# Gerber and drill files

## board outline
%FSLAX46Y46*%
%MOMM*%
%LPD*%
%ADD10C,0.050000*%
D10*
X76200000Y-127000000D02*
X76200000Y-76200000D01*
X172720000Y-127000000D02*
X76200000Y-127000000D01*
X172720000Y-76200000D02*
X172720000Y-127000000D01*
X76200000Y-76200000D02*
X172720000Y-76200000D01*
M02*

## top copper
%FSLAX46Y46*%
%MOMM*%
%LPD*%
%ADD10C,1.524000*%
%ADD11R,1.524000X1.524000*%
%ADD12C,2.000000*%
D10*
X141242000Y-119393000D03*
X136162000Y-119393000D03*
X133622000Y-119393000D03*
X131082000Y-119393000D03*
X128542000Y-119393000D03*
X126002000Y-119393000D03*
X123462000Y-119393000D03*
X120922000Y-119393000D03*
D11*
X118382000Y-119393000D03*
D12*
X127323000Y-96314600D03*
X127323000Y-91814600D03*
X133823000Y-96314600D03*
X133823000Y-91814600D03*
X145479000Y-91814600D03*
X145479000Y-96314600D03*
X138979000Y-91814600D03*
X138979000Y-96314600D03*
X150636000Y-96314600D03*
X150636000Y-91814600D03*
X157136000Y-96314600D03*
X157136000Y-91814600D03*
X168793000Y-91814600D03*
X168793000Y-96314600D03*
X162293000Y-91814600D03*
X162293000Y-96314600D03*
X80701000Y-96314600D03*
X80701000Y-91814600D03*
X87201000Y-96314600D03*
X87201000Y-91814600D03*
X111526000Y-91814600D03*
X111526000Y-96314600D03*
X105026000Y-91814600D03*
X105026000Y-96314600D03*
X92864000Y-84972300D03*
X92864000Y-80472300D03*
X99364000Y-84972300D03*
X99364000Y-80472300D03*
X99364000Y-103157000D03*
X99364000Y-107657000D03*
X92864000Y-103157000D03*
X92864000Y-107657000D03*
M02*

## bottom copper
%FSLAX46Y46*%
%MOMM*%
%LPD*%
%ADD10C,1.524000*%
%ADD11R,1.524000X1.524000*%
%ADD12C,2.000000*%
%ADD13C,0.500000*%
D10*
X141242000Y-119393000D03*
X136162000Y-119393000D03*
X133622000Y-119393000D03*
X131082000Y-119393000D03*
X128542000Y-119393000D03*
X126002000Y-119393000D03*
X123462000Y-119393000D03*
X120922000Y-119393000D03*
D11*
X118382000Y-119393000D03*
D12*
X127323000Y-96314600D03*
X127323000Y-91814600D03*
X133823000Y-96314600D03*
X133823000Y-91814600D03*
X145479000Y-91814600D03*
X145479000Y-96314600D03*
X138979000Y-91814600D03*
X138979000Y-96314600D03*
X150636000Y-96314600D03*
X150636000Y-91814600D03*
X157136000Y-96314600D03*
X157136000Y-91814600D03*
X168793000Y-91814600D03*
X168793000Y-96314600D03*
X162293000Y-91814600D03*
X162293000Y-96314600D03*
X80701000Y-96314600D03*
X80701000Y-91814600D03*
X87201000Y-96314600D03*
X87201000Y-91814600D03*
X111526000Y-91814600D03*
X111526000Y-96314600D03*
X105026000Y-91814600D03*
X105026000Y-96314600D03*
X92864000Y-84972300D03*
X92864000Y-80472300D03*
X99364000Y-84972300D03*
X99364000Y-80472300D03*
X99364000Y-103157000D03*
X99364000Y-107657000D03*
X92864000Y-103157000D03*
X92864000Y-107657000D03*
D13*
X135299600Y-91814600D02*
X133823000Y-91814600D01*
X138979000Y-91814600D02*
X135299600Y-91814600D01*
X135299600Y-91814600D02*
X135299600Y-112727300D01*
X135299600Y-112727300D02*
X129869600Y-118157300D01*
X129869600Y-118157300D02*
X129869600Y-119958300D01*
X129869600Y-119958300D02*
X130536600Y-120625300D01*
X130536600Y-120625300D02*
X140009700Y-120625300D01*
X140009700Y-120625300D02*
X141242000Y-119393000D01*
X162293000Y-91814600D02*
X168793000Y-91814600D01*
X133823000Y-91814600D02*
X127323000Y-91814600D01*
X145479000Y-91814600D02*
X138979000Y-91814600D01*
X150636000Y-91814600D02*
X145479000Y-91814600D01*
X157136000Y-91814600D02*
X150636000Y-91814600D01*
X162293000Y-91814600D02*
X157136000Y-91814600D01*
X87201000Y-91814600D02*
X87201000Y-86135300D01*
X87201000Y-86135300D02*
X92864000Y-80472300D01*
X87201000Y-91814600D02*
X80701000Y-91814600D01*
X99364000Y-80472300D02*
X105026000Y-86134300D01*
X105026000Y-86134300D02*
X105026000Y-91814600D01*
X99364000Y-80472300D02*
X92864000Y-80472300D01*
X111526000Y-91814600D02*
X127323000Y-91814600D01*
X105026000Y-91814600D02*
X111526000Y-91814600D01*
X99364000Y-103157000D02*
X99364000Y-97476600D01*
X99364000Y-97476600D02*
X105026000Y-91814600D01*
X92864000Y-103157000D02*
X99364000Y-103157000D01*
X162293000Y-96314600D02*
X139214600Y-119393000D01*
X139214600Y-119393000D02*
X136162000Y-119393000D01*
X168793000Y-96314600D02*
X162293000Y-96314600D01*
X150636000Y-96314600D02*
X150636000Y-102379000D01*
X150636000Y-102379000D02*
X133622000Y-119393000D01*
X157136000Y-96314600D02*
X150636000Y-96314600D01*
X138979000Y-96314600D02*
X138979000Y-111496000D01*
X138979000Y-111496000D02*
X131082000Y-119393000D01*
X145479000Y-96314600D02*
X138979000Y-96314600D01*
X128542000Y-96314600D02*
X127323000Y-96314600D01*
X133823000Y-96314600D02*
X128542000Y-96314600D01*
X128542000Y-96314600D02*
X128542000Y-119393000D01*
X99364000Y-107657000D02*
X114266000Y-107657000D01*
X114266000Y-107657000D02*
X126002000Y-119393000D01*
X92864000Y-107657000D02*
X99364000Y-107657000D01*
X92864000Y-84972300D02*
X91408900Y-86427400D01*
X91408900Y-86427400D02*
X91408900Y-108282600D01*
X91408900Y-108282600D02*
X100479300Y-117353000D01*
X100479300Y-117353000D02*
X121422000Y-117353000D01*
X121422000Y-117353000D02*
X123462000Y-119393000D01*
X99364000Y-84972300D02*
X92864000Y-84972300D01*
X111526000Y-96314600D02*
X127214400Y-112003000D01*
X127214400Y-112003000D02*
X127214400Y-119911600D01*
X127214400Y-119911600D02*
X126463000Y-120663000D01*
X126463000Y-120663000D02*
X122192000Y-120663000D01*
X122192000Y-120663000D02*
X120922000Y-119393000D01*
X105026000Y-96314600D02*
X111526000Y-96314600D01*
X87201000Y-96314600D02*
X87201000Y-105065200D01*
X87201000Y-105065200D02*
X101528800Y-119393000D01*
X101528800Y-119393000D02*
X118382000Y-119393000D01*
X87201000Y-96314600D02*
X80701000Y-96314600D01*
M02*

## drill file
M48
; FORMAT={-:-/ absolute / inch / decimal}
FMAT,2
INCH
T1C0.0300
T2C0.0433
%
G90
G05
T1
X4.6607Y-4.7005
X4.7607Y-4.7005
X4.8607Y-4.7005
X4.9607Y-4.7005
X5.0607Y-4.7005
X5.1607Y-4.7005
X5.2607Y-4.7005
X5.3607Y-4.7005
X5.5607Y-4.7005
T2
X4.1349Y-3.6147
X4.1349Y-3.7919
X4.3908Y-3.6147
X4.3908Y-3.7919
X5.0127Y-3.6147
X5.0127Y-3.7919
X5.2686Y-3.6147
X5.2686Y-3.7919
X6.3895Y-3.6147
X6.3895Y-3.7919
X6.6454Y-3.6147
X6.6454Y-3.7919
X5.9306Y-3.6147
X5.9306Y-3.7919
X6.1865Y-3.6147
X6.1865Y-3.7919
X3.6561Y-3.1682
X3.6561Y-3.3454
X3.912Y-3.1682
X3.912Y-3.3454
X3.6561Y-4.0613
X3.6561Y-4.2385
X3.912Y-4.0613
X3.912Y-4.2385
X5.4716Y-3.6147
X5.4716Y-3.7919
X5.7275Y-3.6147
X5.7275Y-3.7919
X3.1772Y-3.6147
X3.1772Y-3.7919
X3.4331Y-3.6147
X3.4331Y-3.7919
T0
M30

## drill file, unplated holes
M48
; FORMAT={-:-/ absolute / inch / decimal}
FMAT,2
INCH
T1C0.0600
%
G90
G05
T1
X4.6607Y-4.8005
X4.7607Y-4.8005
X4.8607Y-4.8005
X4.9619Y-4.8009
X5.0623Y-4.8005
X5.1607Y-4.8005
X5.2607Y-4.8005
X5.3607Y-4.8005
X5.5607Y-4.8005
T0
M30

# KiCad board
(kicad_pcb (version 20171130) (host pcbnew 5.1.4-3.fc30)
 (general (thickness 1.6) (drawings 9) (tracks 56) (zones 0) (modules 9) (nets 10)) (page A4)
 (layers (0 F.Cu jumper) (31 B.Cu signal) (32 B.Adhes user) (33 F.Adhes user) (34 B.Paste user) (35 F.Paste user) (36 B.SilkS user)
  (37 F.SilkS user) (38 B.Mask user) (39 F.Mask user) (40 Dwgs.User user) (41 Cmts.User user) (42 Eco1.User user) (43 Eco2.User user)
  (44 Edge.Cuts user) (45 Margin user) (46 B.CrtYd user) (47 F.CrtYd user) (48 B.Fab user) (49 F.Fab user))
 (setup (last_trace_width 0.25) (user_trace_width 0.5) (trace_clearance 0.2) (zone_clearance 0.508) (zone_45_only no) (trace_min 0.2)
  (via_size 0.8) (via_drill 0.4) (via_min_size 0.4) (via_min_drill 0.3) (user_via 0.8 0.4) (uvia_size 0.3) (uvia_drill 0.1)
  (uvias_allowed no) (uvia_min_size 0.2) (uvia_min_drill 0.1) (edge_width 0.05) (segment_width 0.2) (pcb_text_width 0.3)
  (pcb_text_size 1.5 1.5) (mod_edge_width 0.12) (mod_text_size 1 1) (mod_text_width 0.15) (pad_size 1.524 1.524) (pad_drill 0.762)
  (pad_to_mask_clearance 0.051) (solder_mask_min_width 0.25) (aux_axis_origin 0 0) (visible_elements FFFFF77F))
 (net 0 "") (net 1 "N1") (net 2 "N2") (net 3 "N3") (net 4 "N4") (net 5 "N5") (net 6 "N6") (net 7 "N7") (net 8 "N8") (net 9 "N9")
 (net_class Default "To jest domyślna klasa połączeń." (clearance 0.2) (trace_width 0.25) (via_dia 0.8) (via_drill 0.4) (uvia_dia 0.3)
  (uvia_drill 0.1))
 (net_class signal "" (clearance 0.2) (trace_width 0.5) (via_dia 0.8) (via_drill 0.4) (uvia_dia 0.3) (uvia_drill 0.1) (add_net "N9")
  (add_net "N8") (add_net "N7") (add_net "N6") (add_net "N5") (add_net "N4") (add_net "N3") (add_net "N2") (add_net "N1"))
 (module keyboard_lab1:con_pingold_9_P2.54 (layer F.Cu) (at 118.382 119.393)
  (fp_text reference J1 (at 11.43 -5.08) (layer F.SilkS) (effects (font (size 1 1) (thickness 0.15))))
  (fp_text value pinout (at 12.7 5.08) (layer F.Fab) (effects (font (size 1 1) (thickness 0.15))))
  (pad "" np_thru_hole circle (at 22.86 2.54) (size 1.524 1.524) (drill 1.524) (layers *.Cu *.Mask))
  (pad "" np_thru_hole circle (at 17.78 2.54) (size 1.524 1.524) (drill 1.524) (layers *.Cu *.Mask))
  (pad "" np_thru_hole circle (at 15.24 2.54) (size 1.524 1.524) (drill 1.524) (layers *.Cu *.Mask))
  (pad "" np_thru_hole circle (at 12.7 2.54) (size 1.524 1.524) (drill 1.524) (layers *.Cu *.Mask))
  (pad "" np_thru_hole circle (at 10.2 2.54) (size 1.524 1.524) (drill 1.524) (layers *.Cu *.Mask))
  (pad "" np_thru_hole circle (at 7.65 2.55) (size 1.524 1.524) (drill 1.524) (layers *.Cu *.Mask))
  (pad "" np_thru_hole circle (at 5.08 2.54) (size 1.524 1.524) (drill 1.524) (layers *.Cu *.Mask))
  (pad "" np_thru_hole circle (at 2.54 2.54) (size 1.524 1.524) (drill 1.524) (layers *.Cu *.Mask))
  (pad "" np_thru_hole circle (at 0 2.54) (size 1.524 1.524) (drill 1.524) (layers *.Cu *.Mask))
  (pad 9 thru_hole circle (at 22.86 0) (size 1.524 1.524) (drill 0.762) (layers *.Cu *.Mask) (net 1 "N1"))
  (pad 8 thru_hole circle (at 17.78 0) (size 1.524 1.524) (drill 0.762) (layers *.Cu *.Mask) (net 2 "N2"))
  (pad 7 thru_hole circle (at 15.24 0) (size 1.524 1.524) (drill 0.762) (layers *.Cu *.Mask) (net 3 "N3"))
  (pad 6 thru_hole circle (at 12.7 0) (size 1.524 1.524) (drill 0.762) (layers *.Cu *.Mask) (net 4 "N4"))
  (pad 5 thru_hole circle (at 10.16 0) (size 1.524 1.524) (drill 0.762) (layers *.Cu *.Mask) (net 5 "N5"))
  (pad 4 thru_hole circle (at 7.62 0) (size 1.524 1.524) (drill 0.762) (layers *.Cu *.Mask) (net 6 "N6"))
  (pad 3 thru_hole circle (at 5.08 0) (size 1.524 1.524) (drill 0.762) (layers *.Cu *.Mask) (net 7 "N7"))
  (pad 2 thru_hole circle (at 2.54 0) (size 1.524 1.524) (drill 0.762) (layers *.Cu *.Mask) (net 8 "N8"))
  (pad 1 thru_hole rect (at 0 0) (size 1.524 1.524) (drill 0.762) (layers *.Cu *.Mask) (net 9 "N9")))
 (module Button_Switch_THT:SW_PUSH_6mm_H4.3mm (layer F.Cu) (at 127.323 91.8146)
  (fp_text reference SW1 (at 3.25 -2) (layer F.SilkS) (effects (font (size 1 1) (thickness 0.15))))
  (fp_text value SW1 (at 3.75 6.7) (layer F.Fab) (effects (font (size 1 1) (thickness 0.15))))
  (pad 2 thru_hole circle (at 0 4.5 90) (size 2 2) (drill 1.1) (layers *.Cu *.Mask) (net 5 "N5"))
  (pad 1 thru_hole circle (at 0 0 90) (size 2 2) (drill 1.1) (layers *.Cu *.Mask) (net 1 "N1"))
  (pad 2 thru_hole circle (at 6.5 4.5 90) (size 2 2) (drill 1.1) (layers *.Cu *.Mask) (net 5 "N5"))
  (pad 1 thru_hole circle (at 6.5 0 90) (size 2 2) (drill 1.1) (layers *.Cu *.Mask) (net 1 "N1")))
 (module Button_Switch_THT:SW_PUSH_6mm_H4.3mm (layer F.Cu) (at 138.979 91.8146)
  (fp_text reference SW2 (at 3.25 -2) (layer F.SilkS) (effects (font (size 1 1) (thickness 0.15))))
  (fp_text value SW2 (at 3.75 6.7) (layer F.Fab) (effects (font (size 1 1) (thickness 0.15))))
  (pad 1 thru_hole circle (at 6.5 0 90) (size 2 2) (drill 1.1) (layers *.Cu *.Mask) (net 1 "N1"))
  (pad 2 thru_hole circle (at 6.5 4.5 90) (size 2 2) (drill 1.1) (layers *.Cu *.Mask) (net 4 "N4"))
  (pad 1 thru_hole circle (at 0 0 90) (size 2 2) (drill 1.1) (layers *.Cu *.Mask) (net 1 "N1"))
  (pad 2 thru_hole circle (at 0 4.5 90) (size 2 2) (drill 1.1) (layers *.Cu *.Mask) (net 4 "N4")))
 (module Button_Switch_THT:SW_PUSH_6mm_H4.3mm (layer F.Cu) (at 150.636 91.8146)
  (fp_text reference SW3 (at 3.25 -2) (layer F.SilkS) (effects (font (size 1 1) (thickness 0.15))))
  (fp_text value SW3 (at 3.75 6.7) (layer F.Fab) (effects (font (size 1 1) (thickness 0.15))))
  (pad 2 thru_hole circle (at 0 4.5 90) (size 2 2) (drill 1.1) (layers *.Cu *.Mask) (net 3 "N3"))
  (pad 1 thru_hole circle (at 0 0 90) (size 2 2) (drill 1.1) (layers *.Cu *.Mask) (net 1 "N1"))
  (pad 2 thru_hole circle (at 6.5 4.5 90) (size 2 2) (drill 1.1) (layers *.Cu *.Mask) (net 3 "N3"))
  (pad 1 thru_hole circle (at 6.5 0 90) (size 2 2) (drill 1.1) (layers *.Cu *.Mask) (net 1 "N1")))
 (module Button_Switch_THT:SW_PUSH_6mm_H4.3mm (layer F.Cu) (at 162.293 91.8146)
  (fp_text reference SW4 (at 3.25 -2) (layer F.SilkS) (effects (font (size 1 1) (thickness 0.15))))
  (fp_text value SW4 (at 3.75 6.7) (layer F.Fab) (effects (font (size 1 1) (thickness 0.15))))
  (pad 1 thru_hole circle (at 6.5 0 90) (size 2 2) (drill 1.1) (layers *.Cu *.Mask) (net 1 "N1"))
  (pad 2 thru_hole circle (at 6.5 4.5 90) (size 2 2) (drill 1.1) (layers *.Cu *.Mask) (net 2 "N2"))
  (pad 1 thru_hole circle (at 0 0 90) (size 2 2) (drill 1.1) (layers *.Cu *.Mask) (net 1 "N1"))
  (pad 2 thru_hole circle (at 0 4.5 90) (size 2 2) (drill 1.1) (layers *.Cu *.Mask) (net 2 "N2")))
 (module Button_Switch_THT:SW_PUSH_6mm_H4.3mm (layer F.Cu) (at 80.701 91.8146)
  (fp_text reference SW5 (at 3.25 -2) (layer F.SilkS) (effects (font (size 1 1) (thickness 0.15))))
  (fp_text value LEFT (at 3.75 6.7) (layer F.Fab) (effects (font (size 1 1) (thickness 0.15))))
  (pad 2 thru_hole circle (at 0 4.5 90) (size 2 2) (drill 1.1) (layers *.Cu *.Mask) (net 9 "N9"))
  (pad 1 thru_hole circle (at 0 0 90) (size 2 2) (drill 1.1) (layers *.Cu *.Mask) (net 1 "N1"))
  (pad 2 thru_hole circle (at 6.5 4.5 90) (size 2 2) (drill 1.1) (layers *.Cu *.Mask) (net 9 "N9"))
  (pad 1 thru_hole circle (at 6.5 0 90) (size 2 2) (drill 1.1) (layers *.Cu *.Mask) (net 1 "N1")))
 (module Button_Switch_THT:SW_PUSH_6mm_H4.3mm (layer F.Cu) (at 105.026 91.8146)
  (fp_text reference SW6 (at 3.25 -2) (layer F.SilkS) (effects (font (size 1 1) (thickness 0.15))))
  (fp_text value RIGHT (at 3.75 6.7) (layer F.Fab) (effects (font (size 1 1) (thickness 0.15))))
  (pad 1 thru_hole circle (at 6.5 0 90) (size 2 2) (drill 1.1) (layers *.Cu *.Mask) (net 1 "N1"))
  (pad 2 thru_hole circle (at 6.5 4.5 90) (size 2 2) (drill 1.1) (layers *.Cu *.Mask) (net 8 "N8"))
  (pad 1 thru_hole circle (at 0 0 90) (size 2 2) (drill 1.1) (layers *.Cu *.Mask) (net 1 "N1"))
  (pad 2 thru_hole circle (at 0 4.5 90) (size 2 2) (drill 1.1) (layers *.Cu *.Mask) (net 8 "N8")))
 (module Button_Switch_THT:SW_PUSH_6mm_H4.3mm (layer F.Cu) (at 92.864 80.4723)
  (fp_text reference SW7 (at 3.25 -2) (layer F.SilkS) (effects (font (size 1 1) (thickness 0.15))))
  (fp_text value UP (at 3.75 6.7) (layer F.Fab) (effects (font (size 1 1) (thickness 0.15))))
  (pad 2 thru_hole circle (at 0 4.5 90) (size 2 2) (drill 1.1) (layers *.Cu *.Mask) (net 7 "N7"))
  (pad 1 thru_hole circle (at 0 0 90) (size 2 2) (drill 1.1) (layers *.Cu *.Mask) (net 1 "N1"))
  (pad 2 thru_hole circle (at 6.5 4.5 90) (size 2 2) (drill 1.1) (layers *.Cu *.Mask) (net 7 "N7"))
  (pad 1 thru_hole circle (at 6.5 0 90) (size 2 2) (drill 1.1) (layers *.Cu *.Mask) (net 1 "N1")))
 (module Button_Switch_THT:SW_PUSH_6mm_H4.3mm (layer F.Cu) (at 92.864 103.157)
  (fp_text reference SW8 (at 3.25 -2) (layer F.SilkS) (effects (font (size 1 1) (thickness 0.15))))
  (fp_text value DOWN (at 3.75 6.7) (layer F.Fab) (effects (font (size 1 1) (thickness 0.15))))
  (pad 1 thru_hole circle (at 6.5 0 90) (size 2 2) (drill 1.1) (layers *.Cu *.Mask) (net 1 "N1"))
  (pad 2 thru_hole circle (at 6.5 4.5 90) (size 2 2) (drill 1.1) (layers *.Cu *.Mask) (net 6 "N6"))
  (pad 1 thru_hole circle (at 0 0 90) (size 2 2) (drill 1.1) (layers *.Cu *.Mask) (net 1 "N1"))
  (pad 2 thru_hole circle (at 0 4.5 90) (size 2 2) (drill 1.1) (layers *.Cu *.Mask) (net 6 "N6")))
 (gr_line (start 76.2 127) (end 76.2 76.2) (layer Edge.Cuts) (width 0.05))
 (gr_line (start 172.72 127) (end 76.2 127) (layer Edge.Cuts) (width 0.05))
 (gr_line (start 172.72 76.2) (end 172.72 127) (layer Edge.Cuts) (width 0.05))
 (gr_line (start 76.2 76.2) (end 172.72 76.2) (layer Edge.Cuts) (width 0.05))
 (segment (start 135.2996 91.8146) (end 133.823 91.8146) (width 0.5) (layer B.Cu) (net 1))
 (segment (start 138.979 91.8146) (end 135.2996 91.8146) (width 0.5) (layer B.Cu) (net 1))
 (segment (start 135.2996 91.8146) (end 135.2996 112.7273) (width 0.5) (layer B.Cu) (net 1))
 (segment (start 135.2996 112.7273) (end 129.8696 118.1573) (width 0.5) (layer B.Cu) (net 1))
 (segment (start 129.8696 118.1573) (end 129.8696 119.9583) (width 0.5) (layer B.Cu) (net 1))
 (segment (start 129.8696 119.9583) (end 130.5366 120.6253) (width 0.5) (layer B.Cu) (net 1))
 (segment (start 130.5366 120.6253) (end 140.0097 120.6253) (width 0.5) (layer B.Cu) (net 1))
 (segment (start 140.0097 120.6253) (end 141.242 119.393) (width 0.5) (layer B.Cu) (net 1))
 (segment (start 162.293 91.8146) (end 168.793 91.8146) (width 0.5) (layer B.Cu) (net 1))
 (segment (start 133.823 91.8146) (end 127.323 91.8146) (width 0.5) (layer B.Cu) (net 1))
 (segment (start 145.479 91.8146) (end 138.979 91.8146) (width 0.5) (layer B.Cu) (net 1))
 (segment (start 150.636 91.8146) (end 145.479 91.8146) (width 0.5) (layer B.Cu) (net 1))
 (segment (start 157.136 91.8146) (end 150.636 91.8146) (width 0.5) (layer B.Cu) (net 1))
 (segment (start 162.293 91.8146) (end 157.136 91.8146) (width 0.5) (layer B.Cu) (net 1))
 (segment (start 87.201 91.8146) (end 87.201 86.1353) (width 0.5) (layer B.Cu) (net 1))
 (segment (start 87.201 86.1353) (end 92.864 80.4723) (width 0.5) (layer B.Cu) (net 1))
 (segment (start 87.201 91.8146) (end 80.701 91.8146) (width 0.5) (layer B.Cu) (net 1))
 (segment (start 99.364 80.4723) (end 105.026 86.1343) (width 0.5) (layer B.Cu) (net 1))
 (segment (start 105.026 86.1343) (end 105.026 91.8146) (width 0.5) (layer B.Cu) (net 1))
 (segment (start 99.364 80.4723) (end 92.864 80.4723) (width 0.5) (layer B.Cu) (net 1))
 (segment (start 111.526 91.8146) (end 127.323 91.8146) (width 0.5) (layer B.Cu) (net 1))
 (segment (start 105.026 91.8146) (end 111.526 91.8146) (width 0.5) (layer B.Cu) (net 1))
 (segment (start 99.364 103.157) (end 99.364 97.4766) (width 0.5) (layer B.Cu) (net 1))
 (segment (start 99.364 97.4766) (end 105.026 91.8146) (width 0.5) (layer B.Cu) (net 1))
 (segment (start 92.864 103.157) (end 99.364 103.157) (width 0.5) (layer B.Cu) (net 1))
 (segment (start 162.293 96.3146) (end 139.2146 119.393) (width 0.5) (layer B.Cu) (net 2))
 (segment (start 139.2146 119.393) (end 136.162 119.393) (width 0.5) (layer B.Cu) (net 2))
 (segment (start 168.793 96.3146) (end 162.293 96.3146) (width 0.5) (layer B.Cu) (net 2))
 (segment (start 150.636 96.3146) (end 150.636 102.379) (width 0.5) (layer B.Cu) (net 3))
 (segment (start 150.636 102.379) (end 133.622 119.393) (width 0.5) (layer B.Cu) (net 3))
 (segment (start 157.136 96.3146) (end 150.636 96.3146) (width 0.5) (layer B.Cu) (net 3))
 (segment (start 138.979 96.3146) (end 138.979 111.496) (width 0.5) (layer B.Cu) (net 4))
 (segment (start 138.979 111.496) (end 131.082 119.393) (width 0.5) (layer B.Cu) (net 4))
 (segment (start 145.479 96.3146) (end 138.979 96.3146) (width 0.5) (layer B.Cu) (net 4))
 (segment (start 128.542 96.3146) (end 127.323 96.3146) (width 0.5) (layer B.Cu) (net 5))
 (segment (start 133.823 96.3146) (end 128.542 96.3146) (width 0.5) (layer B.Cu) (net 5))
 (segment (start 128.542 96.3146) (end 128.542 119.393) (width 0.5) (layer B.Cu) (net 5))
 (segment (start 99.364 107.657) (end 114.266 107.657) (width 0.5) (layer B.Cu) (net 6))
 (segment (start 114.266 107.657) (end 126.002 119.393) (width 0.5) (layer B.Cu) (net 6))
 (segment (start 92.864 107.657) (end 99.364 107.657) (width 0.5) (layer B.Cu) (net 6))
 (segment (start 92.864 84.9723) (end 91.4089 86.4274) (width 0.5) (layer B.Cu) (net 7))
 (segment (start 91.4089 86.4274) (end 91.4089 108.2826) (width 0.5) (layer B.Cu) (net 7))
 (segment (start 91.4089 108.2826) (end 100.4793 117.353) (width 0.5) (layer B.Cu) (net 7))
 (segment (start 100.4793 117.353) (end 121.422 117.353) (width 0.5) (layer B.Cu) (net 7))
 (segment (start 121.422 117.353) (end 123.462 119.393) (width 0.5) (layer B.Cu) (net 7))
 (segment (start 99.364 84.9723) (end 92.864 84.9723) (width 0.5) (layer B.Cu) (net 7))
 (segment (start 111.526 96.3146) (end 127.2144 112.003) (width 0.5) (layer B.Cu) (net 8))
 (segment (start 127.2144 112.003) (end 127.2144 119.9116) (width 0.5) (layer B.Cu) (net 8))
 (segment (start 127.2144 119.9116) (end 126.463 120.663) (width 0.5) (layer B.Cu) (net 8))
 (segment (start 126.463 120.663) (end 122.192 120.663) (width 0.5) (layer B.Cu) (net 8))
 (segment (start 122.192 120.663) (end 120.922 119.393) (width 0.5) (layer B.Cu) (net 8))
 (segment (start 105.026 96.3146) (end 111.526 96.3146) (width 0.5) (layer B.Cu) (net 8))
 (segment (start 87.201 96.3146) (end 87.201 105.0652) (width 0.5) (layer B.Cu) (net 9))
 (segment (start 87.201 105.0652) (end 101.5288 119.393) (width 0.5) (layer B.Cu) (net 9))
 (segment (start 101.5288 119.393) (end 118.382 119.393) (width 0.5) (layer B.Cu) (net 9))
 (segment (start 87.201 96.3146) (end 80.701 96.3146) (width 0.5) (layer B.Cu) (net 9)))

